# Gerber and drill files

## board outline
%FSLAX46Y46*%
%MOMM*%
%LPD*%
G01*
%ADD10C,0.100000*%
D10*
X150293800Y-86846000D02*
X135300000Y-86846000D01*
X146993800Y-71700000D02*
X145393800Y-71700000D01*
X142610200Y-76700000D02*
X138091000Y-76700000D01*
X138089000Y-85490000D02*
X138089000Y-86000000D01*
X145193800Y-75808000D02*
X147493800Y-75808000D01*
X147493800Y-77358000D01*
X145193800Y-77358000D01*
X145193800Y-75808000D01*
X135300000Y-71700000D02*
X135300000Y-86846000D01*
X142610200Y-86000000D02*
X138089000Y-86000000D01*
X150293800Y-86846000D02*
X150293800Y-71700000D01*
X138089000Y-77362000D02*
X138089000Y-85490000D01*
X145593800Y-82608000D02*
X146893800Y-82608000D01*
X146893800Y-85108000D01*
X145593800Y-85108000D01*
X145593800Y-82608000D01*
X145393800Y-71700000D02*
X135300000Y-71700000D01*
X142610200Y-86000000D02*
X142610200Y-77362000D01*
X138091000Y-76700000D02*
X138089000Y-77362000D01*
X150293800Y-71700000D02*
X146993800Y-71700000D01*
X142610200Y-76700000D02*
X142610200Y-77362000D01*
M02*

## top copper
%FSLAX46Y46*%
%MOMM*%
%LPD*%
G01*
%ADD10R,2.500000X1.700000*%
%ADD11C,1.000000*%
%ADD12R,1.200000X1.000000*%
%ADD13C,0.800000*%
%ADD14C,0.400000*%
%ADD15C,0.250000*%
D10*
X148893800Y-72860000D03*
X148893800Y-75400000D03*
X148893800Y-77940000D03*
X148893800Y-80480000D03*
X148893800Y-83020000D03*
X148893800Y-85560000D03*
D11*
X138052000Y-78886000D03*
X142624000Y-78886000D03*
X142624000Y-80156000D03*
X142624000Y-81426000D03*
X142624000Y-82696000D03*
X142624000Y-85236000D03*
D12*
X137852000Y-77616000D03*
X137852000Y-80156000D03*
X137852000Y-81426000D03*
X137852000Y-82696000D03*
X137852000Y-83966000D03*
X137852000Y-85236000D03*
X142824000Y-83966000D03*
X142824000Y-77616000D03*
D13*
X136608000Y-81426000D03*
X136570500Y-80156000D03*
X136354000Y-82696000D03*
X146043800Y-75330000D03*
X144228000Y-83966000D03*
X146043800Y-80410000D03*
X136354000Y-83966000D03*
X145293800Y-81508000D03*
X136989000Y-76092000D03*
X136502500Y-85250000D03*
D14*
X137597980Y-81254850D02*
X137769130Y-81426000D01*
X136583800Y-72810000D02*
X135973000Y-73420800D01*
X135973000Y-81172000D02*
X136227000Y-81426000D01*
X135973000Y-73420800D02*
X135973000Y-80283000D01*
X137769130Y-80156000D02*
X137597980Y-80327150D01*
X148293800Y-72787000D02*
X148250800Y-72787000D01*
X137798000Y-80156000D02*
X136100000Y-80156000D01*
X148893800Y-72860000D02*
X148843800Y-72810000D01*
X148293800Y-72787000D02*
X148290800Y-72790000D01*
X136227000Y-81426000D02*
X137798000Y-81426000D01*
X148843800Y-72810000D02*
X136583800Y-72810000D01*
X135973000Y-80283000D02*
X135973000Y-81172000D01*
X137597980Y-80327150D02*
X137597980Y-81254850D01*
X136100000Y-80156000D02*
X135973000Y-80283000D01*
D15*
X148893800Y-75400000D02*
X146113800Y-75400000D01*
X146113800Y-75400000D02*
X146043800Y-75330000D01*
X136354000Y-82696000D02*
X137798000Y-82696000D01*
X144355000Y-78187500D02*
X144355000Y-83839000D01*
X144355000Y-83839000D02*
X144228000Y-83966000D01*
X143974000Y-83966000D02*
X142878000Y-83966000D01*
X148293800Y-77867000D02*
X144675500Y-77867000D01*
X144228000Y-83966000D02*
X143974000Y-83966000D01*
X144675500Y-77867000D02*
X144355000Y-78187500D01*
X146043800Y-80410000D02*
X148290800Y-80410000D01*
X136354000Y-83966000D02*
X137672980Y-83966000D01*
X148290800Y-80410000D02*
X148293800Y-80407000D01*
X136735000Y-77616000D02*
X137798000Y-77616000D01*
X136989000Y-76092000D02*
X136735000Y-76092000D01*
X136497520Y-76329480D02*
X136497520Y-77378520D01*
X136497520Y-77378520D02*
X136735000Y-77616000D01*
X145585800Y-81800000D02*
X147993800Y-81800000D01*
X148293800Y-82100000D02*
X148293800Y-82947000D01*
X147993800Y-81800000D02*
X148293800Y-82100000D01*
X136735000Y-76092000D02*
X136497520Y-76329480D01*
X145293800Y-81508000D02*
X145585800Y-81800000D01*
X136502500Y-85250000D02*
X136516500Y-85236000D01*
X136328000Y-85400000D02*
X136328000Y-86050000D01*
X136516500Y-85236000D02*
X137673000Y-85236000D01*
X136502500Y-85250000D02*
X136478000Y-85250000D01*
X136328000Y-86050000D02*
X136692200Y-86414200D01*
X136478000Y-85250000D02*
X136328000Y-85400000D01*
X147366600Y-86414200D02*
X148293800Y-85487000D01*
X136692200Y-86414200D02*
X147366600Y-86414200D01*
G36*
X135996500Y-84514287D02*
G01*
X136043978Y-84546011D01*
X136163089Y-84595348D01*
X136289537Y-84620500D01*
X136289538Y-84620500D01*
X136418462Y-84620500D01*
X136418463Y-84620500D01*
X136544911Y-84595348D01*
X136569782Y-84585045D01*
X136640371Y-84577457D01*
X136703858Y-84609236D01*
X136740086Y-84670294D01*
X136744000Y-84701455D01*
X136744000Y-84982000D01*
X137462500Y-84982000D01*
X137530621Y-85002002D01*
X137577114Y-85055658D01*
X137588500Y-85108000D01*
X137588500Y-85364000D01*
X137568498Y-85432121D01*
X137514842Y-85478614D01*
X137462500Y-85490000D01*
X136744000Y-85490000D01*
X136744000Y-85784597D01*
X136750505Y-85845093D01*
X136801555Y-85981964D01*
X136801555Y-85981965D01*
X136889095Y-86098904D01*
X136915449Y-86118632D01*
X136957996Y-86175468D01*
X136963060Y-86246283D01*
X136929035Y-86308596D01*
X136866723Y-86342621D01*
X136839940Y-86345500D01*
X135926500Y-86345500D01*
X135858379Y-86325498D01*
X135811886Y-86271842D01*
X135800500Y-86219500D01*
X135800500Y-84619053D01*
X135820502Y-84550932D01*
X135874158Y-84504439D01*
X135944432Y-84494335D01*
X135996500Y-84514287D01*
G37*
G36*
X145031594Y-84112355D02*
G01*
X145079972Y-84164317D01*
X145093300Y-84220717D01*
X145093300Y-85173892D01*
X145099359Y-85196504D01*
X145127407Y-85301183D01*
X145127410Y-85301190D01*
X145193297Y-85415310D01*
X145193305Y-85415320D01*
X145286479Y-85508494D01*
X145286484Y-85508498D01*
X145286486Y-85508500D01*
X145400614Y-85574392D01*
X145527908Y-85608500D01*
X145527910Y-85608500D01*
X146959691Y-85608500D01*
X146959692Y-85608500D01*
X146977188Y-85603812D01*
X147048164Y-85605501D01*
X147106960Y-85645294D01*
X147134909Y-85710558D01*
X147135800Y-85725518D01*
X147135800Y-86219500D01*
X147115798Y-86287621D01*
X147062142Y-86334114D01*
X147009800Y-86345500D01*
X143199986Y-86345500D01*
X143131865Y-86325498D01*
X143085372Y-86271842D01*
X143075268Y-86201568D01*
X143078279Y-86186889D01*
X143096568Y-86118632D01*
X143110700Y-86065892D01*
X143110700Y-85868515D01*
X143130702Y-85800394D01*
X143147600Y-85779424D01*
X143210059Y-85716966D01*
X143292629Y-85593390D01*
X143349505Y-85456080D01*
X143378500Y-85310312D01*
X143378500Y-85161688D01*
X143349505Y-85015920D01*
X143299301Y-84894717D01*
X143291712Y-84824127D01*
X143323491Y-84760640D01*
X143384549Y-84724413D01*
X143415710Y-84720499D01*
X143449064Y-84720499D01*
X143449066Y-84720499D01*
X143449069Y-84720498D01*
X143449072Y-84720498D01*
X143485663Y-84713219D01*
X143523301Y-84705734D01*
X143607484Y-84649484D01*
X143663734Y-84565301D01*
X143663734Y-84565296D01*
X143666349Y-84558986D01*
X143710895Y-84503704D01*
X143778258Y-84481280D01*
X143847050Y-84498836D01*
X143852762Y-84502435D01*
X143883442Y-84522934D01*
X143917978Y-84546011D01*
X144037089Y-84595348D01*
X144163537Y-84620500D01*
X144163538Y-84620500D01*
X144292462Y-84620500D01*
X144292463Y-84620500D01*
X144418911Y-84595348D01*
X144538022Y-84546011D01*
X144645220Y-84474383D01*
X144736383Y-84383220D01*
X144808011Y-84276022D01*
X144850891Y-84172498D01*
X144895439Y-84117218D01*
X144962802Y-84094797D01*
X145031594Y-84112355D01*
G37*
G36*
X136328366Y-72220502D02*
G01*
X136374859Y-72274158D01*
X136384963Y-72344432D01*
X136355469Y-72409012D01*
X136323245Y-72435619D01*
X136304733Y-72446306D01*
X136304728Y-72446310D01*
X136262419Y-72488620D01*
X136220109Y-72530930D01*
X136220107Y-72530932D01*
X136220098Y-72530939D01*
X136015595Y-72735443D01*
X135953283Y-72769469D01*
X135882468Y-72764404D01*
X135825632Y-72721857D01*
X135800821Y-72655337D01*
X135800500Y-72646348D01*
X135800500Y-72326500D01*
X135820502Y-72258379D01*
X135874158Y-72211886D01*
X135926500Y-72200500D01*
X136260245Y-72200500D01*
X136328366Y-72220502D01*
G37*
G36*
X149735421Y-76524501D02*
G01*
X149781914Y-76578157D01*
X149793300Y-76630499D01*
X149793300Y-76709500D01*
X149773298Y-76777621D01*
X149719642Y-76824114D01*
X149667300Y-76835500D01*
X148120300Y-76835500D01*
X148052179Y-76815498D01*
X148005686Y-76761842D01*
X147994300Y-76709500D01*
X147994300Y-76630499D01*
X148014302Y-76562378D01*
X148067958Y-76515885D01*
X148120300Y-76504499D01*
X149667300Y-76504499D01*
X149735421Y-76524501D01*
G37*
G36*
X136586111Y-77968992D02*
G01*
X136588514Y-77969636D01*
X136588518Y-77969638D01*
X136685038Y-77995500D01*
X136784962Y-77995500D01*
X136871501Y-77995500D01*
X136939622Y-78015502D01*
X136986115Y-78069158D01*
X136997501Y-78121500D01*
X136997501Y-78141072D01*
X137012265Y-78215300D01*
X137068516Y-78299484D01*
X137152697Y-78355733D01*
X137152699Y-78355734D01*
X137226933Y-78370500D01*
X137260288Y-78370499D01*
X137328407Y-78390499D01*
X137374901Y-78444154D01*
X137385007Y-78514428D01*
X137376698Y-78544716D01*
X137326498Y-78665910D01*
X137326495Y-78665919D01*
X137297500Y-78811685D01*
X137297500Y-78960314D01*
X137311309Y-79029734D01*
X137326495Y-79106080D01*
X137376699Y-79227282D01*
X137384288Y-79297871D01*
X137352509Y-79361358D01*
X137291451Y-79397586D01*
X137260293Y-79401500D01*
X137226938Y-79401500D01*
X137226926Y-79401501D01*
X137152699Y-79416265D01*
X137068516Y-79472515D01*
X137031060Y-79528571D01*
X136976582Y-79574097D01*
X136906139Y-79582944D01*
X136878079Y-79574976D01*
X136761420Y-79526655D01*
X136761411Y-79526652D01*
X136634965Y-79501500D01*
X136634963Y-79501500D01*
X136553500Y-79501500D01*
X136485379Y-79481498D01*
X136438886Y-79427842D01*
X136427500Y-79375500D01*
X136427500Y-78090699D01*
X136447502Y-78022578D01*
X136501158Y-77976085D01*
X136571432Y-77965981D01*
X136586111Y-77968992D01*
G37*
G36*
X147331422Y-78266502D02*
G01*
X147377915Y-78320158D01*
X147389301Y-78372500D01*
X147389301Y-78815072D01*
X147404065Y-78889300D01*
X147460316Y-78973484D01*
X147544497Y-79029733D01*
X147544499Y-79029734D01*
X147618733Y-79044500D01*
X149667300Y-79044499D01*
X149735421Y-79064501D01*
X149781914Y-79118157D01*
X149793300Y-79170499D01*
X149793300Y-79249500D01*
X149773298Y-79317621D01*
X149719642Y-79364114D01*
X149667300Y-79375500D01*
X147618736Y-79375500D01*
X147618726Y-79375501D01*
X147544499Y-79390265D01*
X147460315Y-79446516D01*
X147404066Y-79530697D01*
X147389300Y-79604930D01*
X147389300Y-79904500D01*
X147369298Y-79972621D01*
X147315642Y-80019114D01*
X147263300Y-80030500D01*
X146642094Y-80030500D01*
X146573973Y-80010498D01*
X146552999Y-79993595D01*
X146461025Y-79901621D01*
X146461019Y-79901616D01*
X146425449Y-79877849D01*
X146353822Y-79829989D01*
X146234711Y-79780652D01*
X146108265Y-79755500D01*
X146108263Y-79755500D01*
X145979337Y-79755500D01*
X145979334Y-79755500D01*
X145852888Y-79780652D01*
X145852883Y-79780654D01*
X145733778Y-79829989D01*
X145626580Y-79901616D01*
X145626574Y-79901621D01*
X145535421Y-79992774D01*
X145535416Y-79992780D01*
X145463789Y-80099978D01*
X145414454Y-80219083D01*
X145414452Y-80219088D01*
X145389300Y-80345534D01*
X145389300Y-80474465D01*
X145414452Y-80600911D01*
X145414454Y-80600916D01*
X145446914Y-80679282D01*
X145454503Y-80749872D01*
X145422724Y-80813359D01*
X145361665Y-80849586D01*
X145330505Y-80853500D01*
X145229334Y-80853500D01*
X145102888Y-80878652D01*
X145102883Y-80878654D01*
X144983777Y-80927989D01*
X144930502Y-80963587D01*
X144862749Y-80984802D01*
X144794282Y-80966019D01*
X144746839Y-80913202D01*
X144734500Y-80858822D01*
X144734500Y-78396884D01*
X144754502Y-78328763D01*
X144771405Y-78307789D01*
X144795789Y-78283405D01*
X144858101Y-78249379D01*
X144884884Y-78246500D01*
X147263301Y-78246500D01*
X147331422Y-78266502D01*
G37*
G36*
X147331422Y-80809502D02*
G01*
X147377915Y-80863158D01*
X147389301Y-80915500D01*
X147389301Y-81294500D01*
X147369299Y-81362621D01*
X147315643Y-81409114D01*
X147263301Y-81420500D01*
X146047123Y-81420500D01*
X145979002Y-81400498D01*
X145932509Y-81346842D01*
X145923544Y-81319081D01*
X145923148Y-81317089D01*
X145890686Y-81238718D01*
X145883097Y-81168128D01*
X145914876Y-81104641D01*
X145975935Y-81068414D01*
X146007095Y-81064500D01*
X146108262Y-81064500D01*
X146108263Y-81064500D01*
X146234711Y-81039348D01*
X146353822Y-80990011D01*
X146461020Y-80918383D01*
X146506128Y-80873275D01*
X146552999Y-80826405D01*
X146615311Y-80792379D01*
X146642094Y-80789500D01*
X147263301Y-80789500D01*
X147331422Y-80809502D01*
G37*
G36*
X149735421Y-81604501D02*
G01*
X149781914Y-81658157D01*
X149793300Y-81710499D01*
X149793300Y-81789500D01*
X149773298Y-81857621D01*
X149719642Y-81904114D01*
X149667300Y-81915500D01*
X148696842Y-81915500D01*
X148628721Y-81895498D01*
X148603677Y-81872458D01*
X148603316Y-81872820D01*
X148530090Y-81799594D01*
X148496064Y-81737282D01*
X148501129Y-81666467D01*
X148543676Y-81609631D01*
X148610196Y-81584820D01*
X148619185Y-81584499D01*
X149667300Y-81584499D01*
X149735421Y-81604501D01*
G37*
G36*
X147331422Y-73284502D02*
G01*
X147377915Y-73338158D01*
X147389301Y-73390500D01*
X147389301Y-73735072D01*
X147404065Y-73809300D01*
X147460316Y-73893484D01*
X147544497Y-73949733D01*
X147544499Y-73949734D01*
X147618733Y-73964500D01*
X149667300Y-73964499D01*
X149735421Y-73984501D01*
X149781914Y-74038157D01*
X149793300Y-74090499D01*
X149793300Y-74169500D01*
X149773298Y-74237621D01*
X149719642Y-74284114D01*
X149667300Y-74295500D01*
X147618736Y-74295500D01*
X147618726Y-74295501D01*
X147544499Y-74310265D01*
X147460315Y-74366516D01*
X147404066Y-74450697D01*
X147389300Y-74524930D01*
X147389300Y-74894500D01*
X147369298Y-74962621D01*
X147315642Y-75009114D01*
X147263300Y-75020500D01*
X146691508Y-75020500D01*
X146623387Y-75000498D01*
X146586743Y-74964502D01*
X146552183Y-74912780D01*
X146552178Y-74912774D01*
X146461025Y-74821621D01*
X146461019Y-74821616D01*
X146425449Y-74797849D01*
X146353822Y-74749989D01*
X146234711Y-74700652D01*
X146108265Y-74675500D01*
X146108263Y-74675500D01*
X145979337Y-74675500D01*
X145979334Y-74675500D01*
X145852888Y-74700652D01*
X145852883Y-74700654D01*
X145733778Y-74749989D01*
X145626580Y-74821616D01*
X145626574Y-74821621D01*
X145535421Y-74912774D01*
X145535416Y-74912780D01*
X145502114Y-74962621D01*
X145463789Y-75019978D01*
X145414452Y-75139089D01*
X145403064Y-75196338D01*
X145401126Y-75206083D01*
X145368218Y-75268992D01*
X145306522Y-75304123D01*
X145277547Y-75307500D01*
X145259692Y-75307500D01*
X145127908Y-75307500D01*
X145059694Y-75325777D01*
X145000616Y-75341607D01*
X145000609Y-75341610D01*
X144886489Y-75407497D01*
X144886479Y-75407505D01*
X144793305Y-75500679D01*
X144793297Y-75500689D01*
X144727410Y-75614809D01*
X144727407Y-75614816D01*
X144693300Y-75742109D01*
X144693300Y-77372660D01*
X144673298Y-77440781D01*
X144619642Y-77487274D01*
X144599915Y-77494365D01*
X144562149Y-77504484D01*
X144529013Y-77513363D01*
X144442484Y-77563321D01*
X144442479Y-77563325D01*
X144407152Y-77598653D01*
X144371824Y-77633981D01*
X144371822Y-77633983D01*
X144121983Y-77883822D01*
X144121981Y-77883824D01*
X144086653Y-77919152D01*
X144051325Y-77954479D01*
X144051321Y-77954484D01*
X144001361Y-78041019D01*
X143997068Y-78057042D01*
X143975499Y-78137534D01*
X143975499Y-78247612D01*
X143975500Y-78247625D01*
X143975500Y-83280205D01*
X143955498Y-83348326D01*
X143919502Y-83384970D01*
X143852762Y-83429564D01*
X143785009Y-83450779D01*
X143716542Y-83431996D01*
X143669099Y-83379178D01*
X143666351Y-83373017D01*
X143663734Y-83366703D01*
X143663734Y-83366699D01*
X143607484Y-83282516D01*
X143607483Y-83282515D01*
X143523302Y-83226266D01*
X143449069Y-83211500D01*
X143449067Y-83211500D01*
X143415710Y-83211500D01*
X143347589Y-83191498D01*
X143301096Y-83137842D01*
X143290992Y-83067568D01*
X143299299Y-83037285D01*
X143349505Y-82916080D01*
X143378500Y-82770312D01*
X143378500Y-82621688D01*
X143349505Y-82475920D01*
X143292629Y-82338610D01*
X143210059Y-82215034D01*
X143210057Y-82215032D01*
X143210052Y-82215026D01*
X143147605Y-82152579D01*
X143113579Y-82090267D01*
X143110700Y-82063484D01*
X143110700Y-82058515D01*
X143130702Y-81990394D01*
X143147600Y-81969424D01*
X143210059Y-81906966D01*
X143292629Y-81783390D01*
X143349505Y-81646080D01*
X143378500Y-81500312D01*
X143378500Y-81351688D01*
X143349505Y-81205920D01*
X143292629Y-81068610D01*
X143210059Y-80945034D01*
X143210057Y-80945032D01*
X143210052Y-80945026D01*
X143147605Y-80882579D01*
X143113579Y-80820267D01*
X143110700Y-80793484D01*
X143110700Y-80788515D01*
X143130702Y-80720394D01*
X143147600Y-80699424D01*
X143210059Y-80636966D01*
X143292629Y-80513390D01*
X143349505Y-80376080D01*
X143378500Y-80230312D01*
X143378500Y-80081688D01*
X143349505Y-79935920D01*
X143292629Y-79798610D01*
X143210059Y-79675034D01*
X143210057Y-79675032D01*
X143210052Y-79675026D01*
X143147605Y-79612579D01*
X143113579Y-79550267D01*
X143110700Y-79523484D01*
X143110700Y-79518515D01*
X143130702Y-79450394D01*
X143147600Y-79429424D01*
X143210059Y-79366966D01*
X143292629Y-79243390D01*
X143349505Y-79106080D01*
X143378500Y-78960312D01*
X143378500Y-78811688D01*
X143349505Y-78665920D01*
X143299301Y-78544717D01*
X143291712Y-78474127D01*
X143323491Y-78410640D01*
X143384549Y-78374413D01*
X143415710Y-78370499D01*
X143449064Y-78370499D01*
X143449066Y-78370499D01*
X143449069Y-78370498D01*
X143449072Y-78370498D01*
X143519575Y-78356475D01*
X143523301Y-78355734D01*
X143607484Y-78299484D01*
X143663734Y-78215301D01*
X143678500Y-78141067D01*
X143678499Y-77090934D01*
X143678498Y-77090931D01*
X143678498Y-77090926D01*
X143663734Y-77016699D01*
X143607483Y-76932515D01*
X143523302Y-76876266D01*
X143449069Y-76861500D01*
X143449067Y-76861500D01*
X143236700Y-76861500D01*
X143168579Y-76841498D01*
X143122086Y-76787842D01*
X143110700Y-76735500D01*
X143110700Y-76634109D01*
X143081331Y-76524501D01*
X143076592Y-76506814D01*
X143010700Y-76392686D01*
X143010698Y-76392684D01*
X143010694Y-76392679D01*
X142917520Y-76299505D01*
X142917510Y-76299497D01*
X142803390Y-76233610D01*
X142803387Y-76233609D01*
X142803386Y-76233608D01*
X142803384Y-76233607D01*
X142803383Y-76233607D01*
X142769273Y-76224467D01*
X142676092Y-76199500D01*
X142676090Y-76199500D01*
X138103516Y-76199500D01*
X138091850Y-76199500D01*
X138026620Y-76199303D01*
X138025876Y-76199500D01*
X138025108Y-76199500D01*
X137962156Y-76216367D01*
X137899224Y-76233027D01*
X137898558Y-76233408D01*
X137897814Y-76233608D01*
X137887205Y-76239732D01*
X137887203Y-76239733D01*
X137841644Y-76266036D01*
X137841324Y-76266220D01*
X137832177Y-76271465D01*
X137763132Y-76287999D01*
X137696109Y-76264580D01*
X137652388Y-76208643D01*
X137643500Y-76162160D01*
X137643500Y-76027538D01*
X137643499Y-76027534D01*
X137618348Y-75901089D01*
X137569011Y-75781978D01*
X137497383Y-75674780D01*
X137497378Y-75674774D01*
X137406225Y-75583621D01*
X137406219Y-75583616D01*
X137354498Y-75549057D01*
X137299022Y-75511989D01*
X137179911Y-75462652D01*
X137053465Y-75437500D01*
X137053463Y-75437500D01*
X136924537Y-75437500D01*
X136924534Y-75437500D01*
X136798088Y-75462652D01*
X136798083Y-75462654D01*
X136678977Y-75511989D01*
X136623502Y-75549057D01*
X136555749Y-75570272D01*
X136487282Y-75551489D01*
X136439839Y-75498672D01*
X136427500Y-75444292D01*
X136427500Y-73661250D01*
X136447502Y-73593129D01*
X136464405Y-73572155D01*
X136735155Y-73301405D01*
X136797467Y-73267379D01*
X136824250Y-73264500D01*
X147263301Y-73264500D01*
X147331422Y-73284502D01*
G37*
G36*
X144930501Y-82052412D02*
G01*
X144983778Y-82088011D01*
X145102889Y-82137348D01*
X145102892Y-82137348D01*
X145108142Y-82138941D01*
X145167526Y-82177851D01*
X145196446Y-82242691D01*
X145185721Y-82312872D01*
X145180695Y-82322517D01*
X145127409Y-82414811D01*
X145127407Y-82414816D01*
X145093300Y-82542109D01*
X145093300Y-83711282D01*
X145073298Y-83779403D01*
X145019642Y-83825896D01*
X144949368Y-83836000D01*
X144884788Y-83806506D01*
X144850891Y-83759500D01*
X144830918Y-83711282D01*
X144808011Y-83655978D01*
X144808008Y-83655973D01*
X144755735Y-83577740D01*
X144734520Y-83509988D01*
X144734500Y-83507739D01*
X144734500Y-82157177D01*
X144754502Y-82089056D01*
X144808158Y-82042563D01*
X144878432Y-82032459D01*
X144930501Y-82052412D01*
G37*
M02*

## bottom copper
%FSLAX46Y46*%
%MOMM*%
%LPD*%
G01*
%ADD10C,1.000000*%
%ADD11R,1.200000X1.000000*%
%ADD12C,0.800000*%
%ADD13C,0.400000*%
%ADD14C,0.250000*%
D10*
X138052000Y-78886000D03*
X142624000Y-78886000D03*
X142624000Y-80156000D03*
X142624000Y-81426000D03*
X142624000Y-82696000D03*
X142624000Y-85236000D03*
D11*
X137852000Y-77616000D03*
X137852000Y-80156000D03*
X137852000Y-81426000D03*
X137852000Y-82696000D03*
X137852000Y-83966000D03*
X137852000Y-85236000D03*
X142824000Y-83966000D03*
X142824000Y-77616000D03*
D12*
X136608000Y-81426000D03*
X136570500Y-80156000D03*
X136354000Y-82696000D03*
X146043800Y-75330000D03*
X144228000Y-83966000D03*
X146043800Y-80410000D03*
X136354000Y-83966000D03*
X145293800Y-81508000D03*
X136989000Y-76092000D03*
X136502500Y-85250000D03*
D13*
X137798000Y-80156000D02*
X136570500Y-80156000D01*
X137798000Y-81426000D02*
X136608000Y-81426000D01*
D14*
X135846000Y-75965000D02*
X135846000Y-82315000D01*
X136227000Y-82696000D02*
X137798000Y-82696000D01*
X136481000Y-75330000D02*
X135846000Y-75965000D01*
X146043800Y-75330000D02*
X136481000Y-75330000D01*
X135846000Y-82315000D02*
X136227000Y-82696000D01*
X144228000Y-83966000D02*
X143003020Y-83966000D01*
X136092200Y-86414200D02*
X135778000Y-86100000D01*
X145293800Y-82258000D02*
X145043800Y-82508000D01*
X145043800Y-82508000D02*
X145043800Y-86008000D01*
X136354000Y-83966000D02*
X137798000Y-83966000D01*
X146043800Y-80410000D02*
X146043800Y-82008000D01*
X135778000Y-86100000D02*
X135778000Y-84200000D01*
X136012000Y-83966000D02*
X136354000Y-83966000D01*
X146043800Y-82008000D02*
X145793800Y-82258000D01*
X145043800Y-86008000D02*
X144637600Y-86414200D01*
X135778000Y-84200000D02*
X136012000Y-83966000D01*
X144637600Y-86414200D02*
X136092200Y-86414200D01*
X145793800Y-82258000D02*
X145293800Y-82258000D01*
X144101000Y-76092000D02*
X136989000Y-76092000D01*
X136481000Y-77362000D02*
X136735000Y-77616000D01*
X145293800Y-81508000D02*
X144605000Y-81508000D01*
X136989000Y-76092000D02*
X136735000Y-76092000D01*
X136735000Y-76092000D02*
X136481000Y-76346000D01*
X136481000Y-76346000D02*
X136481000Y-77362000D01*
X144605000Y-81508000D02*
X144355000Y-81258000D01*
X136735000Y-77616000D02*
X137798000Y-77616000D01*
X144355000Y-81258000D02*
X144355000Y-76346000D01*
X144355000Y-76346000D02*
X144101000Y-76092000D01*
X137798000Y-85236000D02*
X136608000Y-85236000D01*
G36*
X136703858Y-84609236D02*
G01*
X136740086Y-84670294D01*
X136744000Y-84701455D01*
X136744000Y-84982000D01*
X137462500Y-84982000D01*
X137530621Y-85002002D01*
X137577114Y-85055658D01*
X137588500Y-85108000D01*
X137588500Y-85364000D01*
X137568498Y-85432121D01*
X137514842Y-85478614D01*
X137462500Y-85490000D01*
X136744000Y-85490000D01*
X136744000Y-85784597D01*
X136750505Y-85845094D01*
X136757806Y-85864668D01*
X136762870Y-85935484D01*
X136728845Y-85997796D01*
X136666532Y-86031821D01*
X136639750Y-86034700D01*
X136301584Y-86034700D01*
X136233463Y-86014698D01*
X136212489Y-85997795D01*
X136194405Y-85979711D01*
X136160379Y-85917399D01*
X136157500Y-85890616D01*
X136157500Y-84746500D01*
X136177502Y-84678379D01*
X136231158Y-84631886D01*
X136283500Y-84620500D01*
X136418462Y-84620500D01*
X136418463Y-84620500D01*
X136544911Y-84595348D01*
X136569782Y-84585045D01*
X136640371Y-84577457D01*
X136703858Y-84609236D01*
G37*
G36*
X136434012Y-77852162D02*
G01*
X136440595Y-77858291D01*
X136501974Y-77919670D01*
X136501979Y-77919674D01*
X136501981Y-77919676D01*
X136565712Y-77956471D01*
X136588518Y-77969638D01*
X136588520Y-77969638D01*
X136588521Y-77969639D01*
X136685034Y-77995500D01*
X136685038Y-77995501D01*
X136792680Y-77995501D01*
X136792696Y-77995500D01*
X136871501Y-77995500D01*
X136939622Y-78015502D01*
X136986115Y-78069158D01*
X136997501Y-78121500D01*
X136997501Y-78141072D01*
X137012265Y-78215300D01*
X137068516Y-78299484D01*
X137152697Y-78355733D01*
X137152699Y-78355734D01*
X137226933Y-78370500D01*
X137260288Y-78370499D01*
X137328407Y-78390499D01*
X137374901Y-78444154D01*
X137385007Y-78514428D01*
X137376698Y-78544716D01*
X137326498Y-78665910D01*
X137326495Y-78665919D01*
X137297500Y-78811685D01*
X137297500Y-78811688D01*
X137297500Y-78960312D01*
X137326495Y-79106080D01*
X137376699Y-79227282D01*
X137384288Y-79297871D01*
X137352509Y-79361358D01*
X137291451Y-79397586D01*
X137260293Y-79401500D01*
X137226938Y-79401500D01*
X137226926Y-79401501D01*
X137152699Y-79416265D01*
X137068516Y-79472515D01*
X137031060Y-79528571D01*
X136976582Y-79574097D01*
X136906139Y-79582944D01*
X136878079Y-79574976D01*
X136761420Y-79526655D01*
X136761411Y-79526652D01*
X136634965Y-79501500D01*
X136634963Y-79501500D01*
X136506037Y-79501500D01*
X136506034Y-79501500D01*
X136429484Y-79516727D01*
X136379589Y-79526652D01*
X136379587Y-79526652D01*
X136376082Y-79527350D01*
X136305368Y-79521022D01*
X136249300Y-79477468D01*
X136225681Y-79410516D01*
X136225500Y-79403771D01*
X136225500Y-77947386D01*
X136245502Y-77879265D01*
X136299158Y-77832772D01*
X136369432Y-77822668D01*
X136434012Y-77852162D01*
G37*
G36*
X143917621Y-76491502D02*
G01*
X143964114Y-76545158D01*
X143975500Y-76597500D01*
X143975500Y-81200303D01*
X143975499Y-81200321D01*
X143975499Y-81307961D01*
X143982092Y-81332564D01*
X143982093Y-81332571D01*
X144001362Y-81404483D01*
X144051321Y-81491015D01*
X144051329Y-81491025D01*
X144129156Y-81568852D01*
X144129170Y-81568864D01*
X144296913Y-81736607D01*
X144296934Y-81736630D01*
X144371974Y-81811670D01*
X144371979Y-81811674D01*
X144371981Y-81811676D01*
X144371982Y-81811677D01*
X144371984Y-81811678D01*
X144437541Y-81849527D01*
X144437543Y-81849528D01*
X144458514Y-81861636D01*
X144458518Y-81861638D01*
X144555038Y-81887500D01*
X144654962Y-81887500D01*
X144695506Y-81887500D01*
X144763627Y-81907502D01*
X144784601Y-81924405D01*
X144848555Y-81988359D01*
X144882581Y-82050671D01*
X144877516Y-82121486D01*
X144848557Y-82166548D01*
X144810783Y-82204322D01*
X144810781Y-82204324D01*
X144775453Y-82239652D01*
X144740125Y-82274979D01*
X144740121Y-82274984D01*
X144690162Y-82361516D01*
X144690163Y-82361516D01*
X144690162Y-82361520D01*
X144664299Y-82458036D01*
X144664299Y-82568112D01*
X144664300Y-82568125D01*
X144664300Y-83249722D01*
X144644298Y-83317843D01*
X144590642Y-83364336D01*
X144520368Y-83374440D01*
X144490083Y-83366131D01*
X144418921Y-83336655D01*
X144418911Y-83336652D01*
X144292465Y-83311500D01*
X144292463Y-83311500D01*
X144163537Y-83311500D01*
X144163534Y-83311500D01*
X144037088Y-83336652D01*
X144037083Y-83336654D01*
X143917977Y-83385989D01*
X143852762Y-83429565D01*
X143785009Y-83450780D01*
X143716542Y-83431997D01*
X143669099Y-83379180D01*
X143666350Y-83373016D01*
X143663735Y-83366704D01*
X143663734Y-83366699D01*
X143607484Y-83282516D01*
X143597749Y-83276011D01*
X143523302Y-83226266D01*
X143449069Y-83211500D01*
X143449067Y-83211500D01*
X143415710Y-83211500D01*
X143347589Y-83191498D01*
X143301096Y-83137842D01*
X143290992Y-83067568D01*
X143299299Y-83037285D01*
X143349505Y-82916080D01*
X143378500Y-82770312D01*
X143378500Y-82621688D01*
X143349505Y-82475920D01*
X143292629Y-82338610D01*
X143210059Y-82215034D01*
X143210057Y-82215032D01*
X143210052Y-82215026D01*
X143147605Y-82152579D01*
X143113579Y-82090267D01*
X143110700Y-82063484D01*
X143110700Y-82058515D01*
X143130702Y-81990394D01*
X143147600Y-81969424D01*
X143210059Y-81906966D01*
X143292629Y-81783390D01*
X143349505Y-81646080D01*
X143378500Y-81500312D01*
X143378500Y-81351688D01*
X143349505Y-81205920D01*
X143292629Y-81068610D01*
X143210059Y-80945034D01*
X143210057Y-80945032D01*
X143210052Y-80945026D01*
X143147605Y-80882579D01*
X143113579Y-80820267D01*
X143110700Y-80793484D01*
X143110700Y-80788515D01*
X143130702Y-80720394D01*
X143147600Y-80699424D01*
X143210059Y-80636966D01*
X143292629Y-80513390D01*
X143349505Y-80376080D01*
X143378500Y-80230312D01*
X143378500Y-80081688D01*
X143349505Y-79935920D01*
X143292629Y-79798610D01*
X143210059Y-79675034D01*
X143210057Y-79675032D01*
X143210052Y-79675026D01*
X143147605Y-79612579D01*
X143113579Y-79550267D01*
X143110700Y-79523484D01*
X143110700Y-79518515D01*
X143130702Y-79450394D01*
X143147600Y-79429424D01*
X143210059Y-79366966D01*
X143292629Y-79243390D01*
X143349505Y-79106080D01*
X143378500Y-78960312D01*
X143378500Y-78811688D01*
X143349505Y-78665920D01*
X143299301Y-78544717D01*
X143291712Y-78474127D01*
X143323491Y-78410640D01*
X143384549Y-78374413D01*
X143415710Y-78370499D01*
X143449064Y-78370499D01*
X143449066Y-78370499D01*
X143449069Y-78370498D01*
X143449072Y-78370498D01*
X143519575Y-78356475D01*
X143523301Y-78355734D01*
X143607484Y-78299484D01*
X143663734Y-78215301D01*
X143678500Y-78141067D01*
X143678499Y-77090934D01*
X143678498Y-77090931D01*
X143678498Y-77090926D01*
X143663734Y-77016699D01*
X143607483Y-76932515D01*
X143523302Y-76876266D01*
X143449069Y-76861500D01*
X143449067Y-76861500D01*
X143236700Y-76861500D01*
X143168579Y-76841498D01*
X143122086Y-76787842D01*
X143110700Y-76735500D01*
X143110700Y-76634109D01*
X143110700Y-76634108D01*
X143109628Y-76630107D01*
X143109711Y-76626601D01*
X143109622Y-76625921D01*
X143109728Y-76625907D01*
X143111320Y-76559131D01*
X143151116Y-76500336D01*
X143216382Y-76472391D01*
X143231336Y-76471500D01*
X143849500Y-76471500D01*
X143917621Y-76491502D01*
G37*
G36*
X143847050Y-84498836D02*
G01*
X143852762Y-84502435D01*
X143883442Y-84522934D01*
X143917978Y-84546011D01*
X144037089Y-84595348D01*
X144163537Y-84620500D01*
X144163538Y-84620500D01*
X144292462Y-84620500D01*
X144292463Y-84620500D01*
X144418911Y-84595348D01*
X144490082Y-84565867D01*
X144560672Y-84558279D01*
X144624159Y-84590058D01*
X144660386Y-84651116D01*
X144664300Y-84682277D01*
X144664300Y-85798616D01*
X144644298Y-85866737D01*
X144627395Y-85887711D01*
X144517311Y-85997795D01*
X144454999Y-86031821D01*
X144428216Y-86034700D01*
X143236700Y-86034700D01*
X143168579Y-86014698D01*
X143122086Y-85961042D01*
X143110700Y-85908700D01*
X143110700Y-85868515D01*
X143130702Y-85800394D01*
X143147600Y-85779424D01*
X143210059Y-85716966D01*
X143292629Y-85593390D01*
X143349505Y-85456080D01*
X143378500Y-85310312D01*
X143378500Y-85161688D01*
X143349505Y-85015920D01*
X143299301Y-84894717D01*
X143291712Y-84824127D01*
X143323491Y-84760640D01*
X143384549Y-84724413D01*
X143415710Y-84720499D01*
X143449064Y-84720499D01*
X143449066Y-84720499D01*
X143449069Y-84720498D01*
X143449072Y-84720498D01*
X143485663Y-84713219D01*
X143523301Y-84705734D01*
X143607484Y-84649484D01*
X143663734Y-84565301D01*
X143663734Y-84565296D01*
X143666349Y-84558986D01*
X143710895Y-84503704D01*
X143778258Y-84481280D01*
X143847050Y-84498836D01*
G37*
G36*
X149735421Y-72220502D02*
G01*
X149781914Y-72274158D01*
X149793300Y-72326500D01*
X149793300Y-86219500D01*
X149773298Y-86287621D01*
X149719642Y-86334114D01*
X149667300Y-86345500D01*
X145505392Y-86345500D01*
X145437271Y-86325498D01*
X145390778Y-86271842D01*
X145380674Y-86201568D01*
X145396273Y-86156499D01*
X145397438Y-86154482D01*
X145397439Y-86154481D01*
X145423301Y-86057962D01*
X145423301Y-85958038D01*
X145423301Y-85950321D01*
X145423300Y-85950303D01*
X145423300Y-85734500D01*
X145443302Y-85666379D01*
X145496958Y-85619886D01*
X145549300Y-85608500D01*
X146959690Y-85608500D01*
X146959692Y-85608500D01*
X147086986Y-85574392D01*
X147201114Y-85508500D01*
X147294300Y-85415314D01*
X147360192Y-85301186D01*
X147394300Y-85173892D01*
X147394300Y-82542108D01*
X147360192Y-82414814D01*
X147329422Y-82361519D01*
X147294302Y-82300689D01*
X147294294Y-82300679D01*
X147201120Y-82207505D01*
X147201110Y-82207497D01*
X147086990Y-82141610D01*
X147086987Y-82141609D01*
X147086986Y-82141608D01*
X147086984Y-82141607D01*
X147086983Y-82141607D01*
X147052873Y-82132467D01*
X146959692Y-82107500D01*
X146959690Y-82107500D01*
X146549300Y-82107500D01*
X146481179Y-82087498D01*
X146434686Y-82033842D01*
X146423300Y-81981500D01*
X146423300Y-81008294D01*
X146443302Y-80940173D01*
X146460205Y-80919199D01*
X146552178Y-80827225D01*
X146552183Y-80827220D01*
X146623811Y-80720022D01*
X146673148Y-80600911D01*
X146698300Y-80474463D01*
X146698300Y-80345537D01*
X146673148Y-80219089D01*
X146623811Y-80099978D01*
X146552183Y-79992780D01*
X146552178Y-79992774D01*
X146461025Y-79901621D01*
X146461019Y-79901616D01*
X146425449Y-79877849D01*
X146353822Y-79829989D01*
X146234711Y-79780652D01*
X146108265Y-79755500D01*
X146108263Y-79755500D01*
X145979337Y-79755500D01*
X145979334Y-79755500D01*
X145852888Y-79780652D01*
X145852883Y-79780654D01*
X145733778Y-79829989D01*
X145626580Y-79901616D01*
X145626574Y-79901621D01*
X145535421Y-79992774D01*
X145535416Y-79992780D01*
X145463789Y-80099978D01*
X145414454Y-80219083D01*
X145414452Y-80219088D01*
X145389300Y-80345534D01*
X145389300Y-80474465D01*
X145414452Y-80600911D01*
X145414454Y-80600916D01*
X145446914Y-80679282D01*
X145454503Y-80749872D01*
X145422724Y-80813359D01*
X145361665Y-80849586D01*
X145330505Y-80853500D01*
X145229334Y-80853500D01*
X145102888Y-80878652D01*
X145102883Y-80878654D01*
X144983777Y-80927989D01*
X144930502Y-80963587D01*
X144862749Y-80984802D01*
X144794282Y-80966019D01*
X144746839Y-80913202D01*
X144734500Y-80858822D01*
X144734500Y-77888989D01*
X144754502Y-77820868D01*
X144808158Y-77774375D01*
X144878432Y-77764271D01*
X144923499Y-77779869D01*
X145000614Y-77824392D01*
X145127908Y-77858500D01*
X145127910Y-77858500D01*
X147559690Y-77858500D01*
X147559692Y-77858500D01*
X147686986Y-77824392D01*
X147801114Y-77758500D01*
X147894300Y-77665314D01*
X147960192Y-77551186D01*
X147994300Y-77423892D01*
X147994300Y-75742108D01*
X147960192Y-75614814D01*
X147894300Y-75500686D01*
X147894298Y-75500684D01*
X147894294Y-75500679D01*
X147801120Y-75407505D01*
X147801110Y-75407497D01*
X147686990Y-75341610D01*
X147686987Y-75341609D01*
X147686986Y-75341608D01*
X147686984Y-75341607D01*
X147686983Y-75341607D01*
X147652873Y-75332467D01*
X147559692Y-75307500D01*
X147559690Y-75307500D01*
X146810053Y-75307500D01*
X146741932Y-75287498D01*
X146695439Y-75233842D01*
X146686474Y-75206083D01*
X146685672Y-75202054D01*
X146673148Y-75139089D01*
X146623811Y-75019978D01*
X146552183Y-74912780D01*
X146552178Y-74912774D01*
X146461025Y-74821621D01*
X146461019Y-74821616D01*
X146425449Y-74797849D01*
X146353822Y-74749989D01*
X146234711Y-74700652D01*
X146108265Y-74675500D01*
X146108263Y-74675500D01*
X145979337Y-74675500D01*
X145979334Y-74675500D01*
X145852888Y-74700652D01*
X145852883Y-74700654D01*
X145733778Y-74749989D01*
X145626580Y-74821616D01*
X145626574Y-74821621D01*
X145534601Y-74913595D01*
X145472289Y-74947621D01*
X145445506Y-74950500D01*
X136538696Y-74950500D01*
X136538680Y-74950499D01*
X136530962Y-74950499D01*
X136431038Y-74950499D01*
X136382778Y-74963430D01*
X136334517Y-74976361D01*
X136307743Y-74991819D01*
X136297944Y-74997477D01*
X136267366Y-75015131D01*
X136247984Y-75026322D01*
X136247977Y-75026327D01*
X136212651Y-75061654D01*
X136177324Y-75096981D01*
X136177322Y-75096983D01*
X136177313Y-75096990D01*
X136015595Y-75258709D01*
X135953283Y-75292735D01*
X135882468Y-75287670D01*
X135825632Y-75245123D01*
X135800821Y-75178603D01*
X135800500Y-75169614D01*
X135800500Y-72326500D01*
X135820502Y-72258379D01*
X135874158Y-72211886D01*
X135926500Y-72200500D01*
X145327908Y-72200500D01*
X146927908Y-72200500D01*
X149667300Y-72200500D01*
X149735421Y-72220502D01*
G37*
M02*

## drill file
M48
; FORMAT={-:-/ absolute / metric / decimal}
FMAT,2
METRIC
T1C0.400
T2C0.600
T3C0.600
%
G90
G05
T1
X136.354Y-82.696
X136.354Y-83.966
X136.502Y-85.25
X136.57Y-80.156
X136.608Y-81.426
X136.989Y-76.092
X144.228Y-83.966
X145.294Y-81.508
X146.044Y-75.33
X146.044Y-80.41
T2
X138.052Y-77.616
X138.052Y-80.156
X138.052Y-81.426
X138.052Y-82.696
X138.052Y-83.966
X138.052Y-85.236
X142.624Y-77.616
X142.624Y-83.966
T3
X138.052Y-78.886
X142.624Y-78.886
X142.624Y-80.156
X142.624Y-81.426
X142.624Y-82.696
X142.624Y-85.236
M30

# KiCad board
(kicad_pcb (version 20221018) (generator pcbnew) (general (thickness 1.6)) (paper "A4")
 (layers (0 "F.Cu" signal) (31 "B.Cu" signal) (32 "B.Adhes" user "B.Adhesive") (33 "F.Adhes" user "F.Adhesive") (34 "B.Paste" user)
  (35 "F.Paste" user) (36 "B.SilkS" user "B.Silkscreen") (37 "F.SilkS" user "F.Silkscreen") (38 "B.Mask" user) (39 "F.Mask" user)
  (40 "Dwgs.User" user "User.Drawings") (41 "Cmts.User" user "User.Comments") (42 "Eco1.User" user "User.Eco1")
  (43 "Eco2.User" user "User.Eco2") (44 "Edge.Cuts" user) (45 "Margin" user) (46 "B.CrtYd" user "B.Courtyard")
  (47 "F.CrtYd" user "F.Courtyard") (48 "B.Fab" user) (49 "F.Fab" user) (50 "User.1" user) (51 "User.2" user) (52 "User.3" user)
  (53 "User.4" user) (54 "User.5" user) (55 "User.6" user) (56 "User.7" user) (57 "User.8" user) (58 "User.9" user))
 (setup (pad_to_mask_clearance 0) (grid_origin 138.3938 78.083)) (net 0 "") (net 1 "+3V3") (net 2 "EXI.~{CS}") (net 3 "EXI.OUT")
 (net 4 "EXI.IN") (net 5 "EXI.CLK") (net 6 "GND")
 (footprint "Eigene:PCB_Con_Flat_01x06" (layer "F.Cu") (at 148.8938 79.21)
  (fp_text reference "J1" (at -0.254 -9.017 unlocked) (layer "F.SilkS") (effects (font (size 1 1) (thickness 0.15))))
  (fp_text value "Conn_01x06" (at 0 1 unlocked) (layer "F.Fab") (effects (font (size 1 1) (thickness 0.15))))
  (pad "1" smd rect (at 0 -6.35) (size 2.5 1.7) (layers "F.Cu" "F.Paste" "F.Mask") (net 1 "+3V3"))
  (pad "2" smd rect (at 0 -3.81) (size 2.5 1.7) (layers "F.Cu" "F.Paste" "F.Mask") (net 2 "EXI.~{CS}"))
  (pad "3" smd rect (at 0 -1.27) (size 2.5 1.7) (layers "F.Cu" "F.Paste" "F.Mask") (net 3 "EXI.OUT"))
  (pad "4" smd rect (at 0 1.27) (size 2.5 1.7) (layers "F.Cu" "F.Paste" "F.Mask") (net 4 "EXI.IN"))
  (pad "5" smd rect (at 0 3.81) (size 2.5 1.7) (layers "F.Cu" "F.Paste" "F.Mask") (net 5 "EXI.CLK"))
  (pad "6" smd rect (at 0 6.35) (size 2.5 1.7) (layers "F.Cu" "F.Paste" "F.Mask") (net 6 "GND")))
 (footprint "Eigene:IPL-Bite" (layer "F.Cu") (at 140.338 81.426)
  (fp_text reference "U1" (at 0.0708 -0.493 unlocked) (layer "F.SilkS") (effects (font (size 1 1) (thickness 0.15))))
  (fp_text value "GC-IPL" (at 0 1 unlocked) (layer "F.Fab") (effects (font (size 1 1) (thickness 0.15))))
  (pad "" np_thru_hole circle (at -2.286 -2.54) (size 1 1) (drill 0.6) (layers "F&B.Cu" "*.Mask"))
  (pad "" np_thru_hole circle (at 2.286 -2.54) (size 1 1) (drill 0.6) (layers "F&B.Cu" "*.Mask"))
  (pad "" np_thru_hole circle (at 2.286 -1.27) (size 1 1) (drill 0.6) (layers "F&B.Cu" "*.Mask"))
  (pad "" np_thru_hole circle (at 2.286 0) (size 1 1) (drill 0.6) (layers "F&B.Cu" "*.Mask"))
  (pad "" np_thru_hole circle (at 2.286 1.27) (size 1 1) (drill 0.6) (layers "F&B.Cu" "*.Mask"))
  (pad "" np_thru_hole circle (at 2.286 3.81) (size 1 1) (drill 0.6) (layers "F&B.Cu" "*.Mask"))
  (pad "1" thru_hole rect (at -2.286 -3.81) (size 1.2 1) (drill 0.6 (offset -0.2 0)) (layers "*.Cu" "*.Mask") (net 5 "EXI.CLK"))
  (pad "3" thru_hole rect (at -2.286 -1.27) (size 1.2 1) (drill 0.6 (offset -0.2 0)) (layers "*.Cu" "*.Mask") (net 1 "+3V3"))
  (pad "4" thru_hole rect (at -2.286 0) (size 1.2 1) (drill 0.6 (offset -0.2 0)) (layers "*.Cu" "*.Mask") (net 1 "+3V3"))
  (pad "5" thru_hole rect (at -2.286 1.27) (size 1.2 1) (drill 0.6 (offset -0.2 0)) (layers "*.Cu" "*.Mask") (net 2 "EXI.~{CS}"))
  (pad "6" thru_hole rect (at -2.286 2.54) (size 1.2 1) (drill 0.6 (offset -0.2 0)) (layers "*.Cu" "*.Mask") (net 4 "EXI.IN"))
  (pad "7" thru_hole rect (at -2.286 3.81) (size 1.2 1) (drill 0.6 (offset -0.2 0)) (layers "*.Cu" "*.Mask") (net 6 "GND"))
  (pad "9" thru_hole rect (at 2.286 2.54 180) (size 1.2 1) (drill 0.6 (offset -0.2 0)) (layers "*.Cu" "*.Mask") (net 3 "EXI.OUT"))
  (pad "14" thru_hole rect (at 2.286 -3.81 180) (size 1.2 1) (drill 0.6 (offset -0.2 0)) (layers "*.Cu" "*.Mask")))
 (gr_line (start 150.2938 86.846) (end 135.3 86.846) (stroke (width 0.1) (type solid)) (layer "Edge.Cuts"))
 (gr_line (start 146.9938 71.7) (end 145.3938 71.7) (stroke (width 0.1) (type solid)) (layer "Edge.Cuts"))
 (gr_line (start 142.6102 76.7) (end 138.091 76.7) (stroke (width 0.1) (type solid)) (layer "Edge.Cuts"))
 (gr_line (start 138.089 85.49) (end 138.089 86) (stroke (width 0.1) (type solid)) (layer "Edge.Cuts"))
 (gr_rect (start 145.1938 75.808) (end 147.4938 77.358) (stroke (width 0.1) (type solid)) (fill none) (layer "Edge.Cuts"))
 (gr_line (start 135.3 71.7) (end 135.3 86.846) (stroke (width 0.1) (type solid)) (layer "Edge.Cuts"))
 (gr_line (start 142.6102 86) (end 138.089 86) (stroke (width 0.1) (type solid)) (layer "Edge.Cuts"))
 (gr_line (start 150.2938 86.846) (end 150.2938 71.7) (stroke (width 0.1) (type solid)) (layer "Edge.Cuts"))
 (gr_line (start 138.089 77.362) (end 138.089 85.49) (stroke (width 0.1) (type solid)) (layer "Edge.Cuts"))
 (gr_rect (start 145.5938 82.608) (end 146.8938 85.108) (stroke (width 0.1) (type solid)) (fill none) (layer "Edge.Cuts"))
 (gr_line (start 145.3938 71.7) (end 135.3 71.7) (stroke (width 0.1) (type solid)) (layer "Edge.Cuts"))
 (gr_line (start 142.6102 86) (end 142.6102 77.362) (stroke (width 0.1) (type solid)) (layer "Edge.Cuts"))
 (gr_line (start 138.091 76.7) (end 138.089 77.362) (stroke (width 0.1) (type solid)) (layer "Edge.Cuts"))
 (gr_line (start 150.2938 71.7) (end 146.9938 71.7) (stroke (width 0.1) (type solid)) (layer "Edge.Cuts"))
 (gr_line (start 142.6102 76.7) (end 142.6102 77.362) (stroke (width 0.1) (type solid)) (layer "Edge.Cuts"))
 (segment (start 137.59798 81.25485) (end 137.76913 81.426) (width 0.4) (layer "F.Cu") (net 1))
 (segment (start 136.5838 72.81) (end 135.973 73.4208) (width 0.4) (layer "F.Cu") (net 1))
 (segment (start 135.973 81.172) (end 136.227 81.426) (width 0.4) (layer "F.Cu") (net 1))
 (segment (start 135.973 73.4208) (end 135.973 80.283) (width 0.4) (layer "F.Cu") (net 1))
 (segment (start 137.76913 80.156) (end 137.59798 80.32715) (width 0.4) (layer "F.Cu") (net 1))
 (segment (start 148.2938 72.787) (end 148.2508 72.787) (width 0.4) (layer "F.Cu") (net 1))
 (segment (start 137.798 80.156) (end 136.1 80.156) (width 0.4) (layer "F.Cu") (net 1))
 (segment (start 148.8938 72.86) (end 148.8438 72.81) (width 0.4) (layer "F.Cu") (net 1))
 (segment (start 148.2938 72.787) (end 148.2908 72.79) (width 0.4) (layer "F.Cu") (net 1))
 (segment (start 136.227 81.426) (end 137.798 81.426) (width 0.4) (layer "F.Cu") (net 1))
 (segment (start 148.8438 72.81) (end 136.5838 72.81) (width 0.4) (layer "F.Cu") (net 1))
 (segment (start 135.973 80.283) (end 135.973 81.172) (width 0.4) (layer "F.Cu") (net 1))
 (segment (start 137.59798 80.32715) (end 137.59798 81.25485) (width 0.4) (layer "F.Cu") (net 1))
 (segment (start 136.1 80.156) (end 135.973 80.283) (width 0.4) (layer "F.Cu") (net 1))
 (via (at 136.608 81.426) (size 0.8) (drill 0.4) (layers "F.Cu" "B.Cu") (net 1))
 (via (at 136.5705 80.156) (size 0.8) (drill 0.4) (layers "F.Cu" "B.Cu") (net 1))
 (segment (start 137.798 80.156) (end 136.5705 80.156) (width 0.4) (layer "B.Cu") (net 1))
 (segment (start 137.798 81.426) (end 136.608 81.426) (width 0.4) (layer "B.Cu") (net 1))
 (segment (start 148.8938 75.4) (end 146.1138 75.4) (width 0.25) (layer "F.Cu") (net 2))
 (segment (start 146.1138 75.4) (end 146.0438 75.33) (width 0.25) (layer "F.Cu") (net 2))
 (segment (start 136.354 82.696) (end 137.798 82.696) (width 0.25) (layer "F.Cu") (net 2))
 (via (at 136.354 82.696) (size 0.8) (drill 0.4) (layers "F.Cu" "B.Cu") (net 2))
 (via (at 146.0438 75.33) (size 0.8) (drill 0.4) (layers "F.Cu" "B.Cu") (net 2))
 (segment (start 135.846 75.965) (end 135.846 82.315) (width 0.25) (layer "B.Cu") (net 2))
 (segment (start 136.227 82.696) (end 137.798 82.696) (width 0.25) (layer "B.Cu") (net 2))
 (segment (start 136.481 75.33) (end 135.846 75.965) (width 0.25) (layer "B.Cu") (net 2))
 (segment (start 146.0438 75.33) (end 136.481 75.33) (width 0.25) (layer "B.Cu") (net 2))
 (segment (start 135.846 82.315) (end 136.227 82.696) (width 0.25) (layer "B.Cu") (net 2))
 (segment (start 144.355 78.1875) (end 144.355 83.839) (width 0.25) (layer "F.Cu") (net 3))
 (segment (start 144.355 83.839) (end 144.228 83.966) (width 0.25) (layer "F.Cu") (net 3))
 (segment (start 143.974 83.966) (end 142.878 83.966) (width 0.25) (layer "F.Cu") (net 3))
 (segment (start 148.2938 77.867) (end 144.6755 77.867) (width 0.25) (layer "F.Cu") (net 3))
 (segment (start 144.228 83.966) (end 143.974 83.966) (width 0.25) (layer "F.Cu") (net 3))
 (segment (start 144.6755 77.867) (end 144.355 78.1875) (width 0.25) (layer "F.Cu") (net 3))
 (via (at 144.228 83.966) (size 0.8) (drill 0.4) (layers "F.Cu" "B.Cu") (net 3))
 (segment (start 144.228 83.966) (end 143.00302 83.966) (width 0.25) (layer "B.Cu") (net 3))
 (segment (start 146.0438 80.41) (end 148.2908 80.41) (width 0.25) (layer "F.Cu") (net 4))
 (segment (start 136.354 83.966) (end 137.67298 83.966) (width 0.25) (layer "F.Cu") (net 4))
 (segment (start 148.2908 80.41) (end 148.2938 80.407) (width 0.25) (layer "F.Cu") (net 4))
 (via (at 146.0438 80.41) (size 0.8) (drill 0.4) (layers "F.Cu" "B.Cu") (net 4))
 (via (at 136.354 83.966) (size 0.8) (drill 0.4) (layers "F.Cu" "B.Cu") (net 4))
 (segment (start 136.0922 86.4142) (end 135.778 86.1) (width 0.25) (layer "B.Cu") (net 4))
 (segment (start 145.2938 82.258) (end 145.0438 82.508) (width 0.25) (layer "B.Cu") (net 4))
 (segment (start 145.0438 82.508) (end 145.0438 86.008) (width 0.25) (layer "B.Cu") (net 4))
 (segment (start 136.354 83.966) (end 137.798 83.966) (width 0.25) (layer "B.Cu") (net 4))
 (segment (start 146.0438 80.41) (end 146.0438 82.008) (width 0.25) (layer "B.Cu") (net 4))
 (segment (start 135.778 86.1) (end 135.778 84.2) (width 0.25) (layer "B.Cu") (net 4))
 (segment (start 136.012 83.966) (end 136.354 83.966) (width 0.25) (layer "B.Cu") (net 4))
 (segment (start 146.0438 82.008) (end 145.7938 82.258) (width 0.25) (layer "B.Cu") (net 4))
 (segment (start 145.0438 86.008) (end 144.6376 86.4142) (width 0.25) (layer "B.Cu") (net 4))
 (segment (start 135.778 84.2) (end 136.012 83.966) (width 0.25) (layer "B.Cu") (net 4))
 (segment (start 144.6376 86.4142) (end 136.0922 86.4142) (width 0.25) (layer "B.Cu") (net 4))
 (segment (start 145.7938 82.258) (end 145.2938 82.258) (width 0.25) (layer "B.Cu") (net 4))
 (segment (start 136.735 77.616) (end 137.798 77.616) (width 0.25) (layer "F.Cu") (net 5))
 (segment (start 136.989 76.092) (end 136.735 76.092) (width 0.25) (layer "F.Cu") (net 5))
 (segment (start 136.49752 76.32948) (end 136.49752 77.37852) (width 0.25) (layer "F.Cu") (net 5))
 (segment (start 136.49752 77.37852) (end 136.735 77.616) (width 0.25) (layer "F.Cu") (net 5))
 (segment (start 145.5858 81.8) (end 147.9938 81.8) (width 0.25) (layer "F.Cu") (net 5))
 (segment (start 148.2938 82.1) (end 148.2938 82.947) (width 0.25) (layer "F.Cu") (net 5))
 (segment (start 147.9938 81.8) (end 148.2938 82.1) (width 0.25) (layer "F.Cu") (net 5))
 (segment (start 136.735 76.092) (end 136.49752 76.32948) (width 0.25) (layer "F.Cu") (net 5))
 (segment (start 145.2938 81.508) (end 145.5858 81.8) (width 0.25) (layer "F.Cu") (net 5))
 (via (at 145.2938 81.508) (size 0.8) (drill 0.4) (layers "F.Cu" "B.Cu") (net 5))
 (via (at 136.989 76.092) (size 0.8) (drill 0.4) (layers "F.Cu" "B.Cu") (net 5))
 (segment (start 144.101 76.092) (end 136.989 76.092) (width 0.25) (layer "B.Cu") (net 5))
 (segment (start 136.481 77.362) (end 136.735 77.616) (width 0.25) (layer "B.Cu") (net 5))
 (segment (start 145.2938 81.508) (end 144.605 81.508) (width 0.25) (layer "B.Cu") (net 5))
 (segment (start 136.989 76.092) (end 136.735 76.092) (width 0.25) (layer "B.Cu") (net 5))
 (segment (start 136.735 76.092) (end 136.481 76.346) (width 0.25) (layer "B.Cu") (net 5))
 (segment (start 136.481 76.346) (end 136.481 77.362) (width 0.25) (layer "B.Cu") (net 5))
 (segment (start 144.605 81.508) (end 144.355 81.258) (width 0.25) (layer "B.Cu") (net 5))
 (segment (start 136.735 77.616) (end 137.798 77.616) (width 0.25) (layer "B.Cu") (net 5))
 (segment (start 144.355 81.258) (end 144.355 76.346) (width 0.25) (layer "B.Cu") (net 5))
 (segment (start 144.355 76.346) (end 144.101 76.092) (width 0.25) (layer "B.Cu") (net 5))
 (segment (start 136.5025 85.25) (end 136.5165 85.236) (width 0.25) (layer "F.Cu") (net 6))
 (segment (start 136.328 85.4) (end 136.328 86.05) (width 0.25) (layer "F.Cu") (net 6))
 (segment (start 136.5165 85.236) (end 137.673 85.236) (width 0.25) (layer "F.Cu") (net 6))
 (segment (start 136.5025 85.25) (end 136.478 85.25) (width 0.25) (layer "F.Cu") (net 6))
 (segment (start 136.328 86.05) (end 136.6922 86.4142) (width 0.25) (layer "F.Cu") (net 6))
 (segment (start 136.478 85.25) (end 136.328 85.4) (width 0.25) (layer "F.Cu") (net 6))
 (segment (start 147.3666 86.4142) (end 148.2938 85.487) (width 0.25) (layer "F.Cu") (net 6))
 (segment (start 136.6922 86.4142) (end 147.3666 86.4142) (width 0.25) (layer "F.Cu") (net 6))
 (via (at 136.5025 85.25) (size 0.8) (drill 0.4) (layers "F.Cu" "B.Cu") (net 6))
 (segment (start 137.798 85.236) (end 136.608 85.236) (width 0.25) (layer "B.Cu") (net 6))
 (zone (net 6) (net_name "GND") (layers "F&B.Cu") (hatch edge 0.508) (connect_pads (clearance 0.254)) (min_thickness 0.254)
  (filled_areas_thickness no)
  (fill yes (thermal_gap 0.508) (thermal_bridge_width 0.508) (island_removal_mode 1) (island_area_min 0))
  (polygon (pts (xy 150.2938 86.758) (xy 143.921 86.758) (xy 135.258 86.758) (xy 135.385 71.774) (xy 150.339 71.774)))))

